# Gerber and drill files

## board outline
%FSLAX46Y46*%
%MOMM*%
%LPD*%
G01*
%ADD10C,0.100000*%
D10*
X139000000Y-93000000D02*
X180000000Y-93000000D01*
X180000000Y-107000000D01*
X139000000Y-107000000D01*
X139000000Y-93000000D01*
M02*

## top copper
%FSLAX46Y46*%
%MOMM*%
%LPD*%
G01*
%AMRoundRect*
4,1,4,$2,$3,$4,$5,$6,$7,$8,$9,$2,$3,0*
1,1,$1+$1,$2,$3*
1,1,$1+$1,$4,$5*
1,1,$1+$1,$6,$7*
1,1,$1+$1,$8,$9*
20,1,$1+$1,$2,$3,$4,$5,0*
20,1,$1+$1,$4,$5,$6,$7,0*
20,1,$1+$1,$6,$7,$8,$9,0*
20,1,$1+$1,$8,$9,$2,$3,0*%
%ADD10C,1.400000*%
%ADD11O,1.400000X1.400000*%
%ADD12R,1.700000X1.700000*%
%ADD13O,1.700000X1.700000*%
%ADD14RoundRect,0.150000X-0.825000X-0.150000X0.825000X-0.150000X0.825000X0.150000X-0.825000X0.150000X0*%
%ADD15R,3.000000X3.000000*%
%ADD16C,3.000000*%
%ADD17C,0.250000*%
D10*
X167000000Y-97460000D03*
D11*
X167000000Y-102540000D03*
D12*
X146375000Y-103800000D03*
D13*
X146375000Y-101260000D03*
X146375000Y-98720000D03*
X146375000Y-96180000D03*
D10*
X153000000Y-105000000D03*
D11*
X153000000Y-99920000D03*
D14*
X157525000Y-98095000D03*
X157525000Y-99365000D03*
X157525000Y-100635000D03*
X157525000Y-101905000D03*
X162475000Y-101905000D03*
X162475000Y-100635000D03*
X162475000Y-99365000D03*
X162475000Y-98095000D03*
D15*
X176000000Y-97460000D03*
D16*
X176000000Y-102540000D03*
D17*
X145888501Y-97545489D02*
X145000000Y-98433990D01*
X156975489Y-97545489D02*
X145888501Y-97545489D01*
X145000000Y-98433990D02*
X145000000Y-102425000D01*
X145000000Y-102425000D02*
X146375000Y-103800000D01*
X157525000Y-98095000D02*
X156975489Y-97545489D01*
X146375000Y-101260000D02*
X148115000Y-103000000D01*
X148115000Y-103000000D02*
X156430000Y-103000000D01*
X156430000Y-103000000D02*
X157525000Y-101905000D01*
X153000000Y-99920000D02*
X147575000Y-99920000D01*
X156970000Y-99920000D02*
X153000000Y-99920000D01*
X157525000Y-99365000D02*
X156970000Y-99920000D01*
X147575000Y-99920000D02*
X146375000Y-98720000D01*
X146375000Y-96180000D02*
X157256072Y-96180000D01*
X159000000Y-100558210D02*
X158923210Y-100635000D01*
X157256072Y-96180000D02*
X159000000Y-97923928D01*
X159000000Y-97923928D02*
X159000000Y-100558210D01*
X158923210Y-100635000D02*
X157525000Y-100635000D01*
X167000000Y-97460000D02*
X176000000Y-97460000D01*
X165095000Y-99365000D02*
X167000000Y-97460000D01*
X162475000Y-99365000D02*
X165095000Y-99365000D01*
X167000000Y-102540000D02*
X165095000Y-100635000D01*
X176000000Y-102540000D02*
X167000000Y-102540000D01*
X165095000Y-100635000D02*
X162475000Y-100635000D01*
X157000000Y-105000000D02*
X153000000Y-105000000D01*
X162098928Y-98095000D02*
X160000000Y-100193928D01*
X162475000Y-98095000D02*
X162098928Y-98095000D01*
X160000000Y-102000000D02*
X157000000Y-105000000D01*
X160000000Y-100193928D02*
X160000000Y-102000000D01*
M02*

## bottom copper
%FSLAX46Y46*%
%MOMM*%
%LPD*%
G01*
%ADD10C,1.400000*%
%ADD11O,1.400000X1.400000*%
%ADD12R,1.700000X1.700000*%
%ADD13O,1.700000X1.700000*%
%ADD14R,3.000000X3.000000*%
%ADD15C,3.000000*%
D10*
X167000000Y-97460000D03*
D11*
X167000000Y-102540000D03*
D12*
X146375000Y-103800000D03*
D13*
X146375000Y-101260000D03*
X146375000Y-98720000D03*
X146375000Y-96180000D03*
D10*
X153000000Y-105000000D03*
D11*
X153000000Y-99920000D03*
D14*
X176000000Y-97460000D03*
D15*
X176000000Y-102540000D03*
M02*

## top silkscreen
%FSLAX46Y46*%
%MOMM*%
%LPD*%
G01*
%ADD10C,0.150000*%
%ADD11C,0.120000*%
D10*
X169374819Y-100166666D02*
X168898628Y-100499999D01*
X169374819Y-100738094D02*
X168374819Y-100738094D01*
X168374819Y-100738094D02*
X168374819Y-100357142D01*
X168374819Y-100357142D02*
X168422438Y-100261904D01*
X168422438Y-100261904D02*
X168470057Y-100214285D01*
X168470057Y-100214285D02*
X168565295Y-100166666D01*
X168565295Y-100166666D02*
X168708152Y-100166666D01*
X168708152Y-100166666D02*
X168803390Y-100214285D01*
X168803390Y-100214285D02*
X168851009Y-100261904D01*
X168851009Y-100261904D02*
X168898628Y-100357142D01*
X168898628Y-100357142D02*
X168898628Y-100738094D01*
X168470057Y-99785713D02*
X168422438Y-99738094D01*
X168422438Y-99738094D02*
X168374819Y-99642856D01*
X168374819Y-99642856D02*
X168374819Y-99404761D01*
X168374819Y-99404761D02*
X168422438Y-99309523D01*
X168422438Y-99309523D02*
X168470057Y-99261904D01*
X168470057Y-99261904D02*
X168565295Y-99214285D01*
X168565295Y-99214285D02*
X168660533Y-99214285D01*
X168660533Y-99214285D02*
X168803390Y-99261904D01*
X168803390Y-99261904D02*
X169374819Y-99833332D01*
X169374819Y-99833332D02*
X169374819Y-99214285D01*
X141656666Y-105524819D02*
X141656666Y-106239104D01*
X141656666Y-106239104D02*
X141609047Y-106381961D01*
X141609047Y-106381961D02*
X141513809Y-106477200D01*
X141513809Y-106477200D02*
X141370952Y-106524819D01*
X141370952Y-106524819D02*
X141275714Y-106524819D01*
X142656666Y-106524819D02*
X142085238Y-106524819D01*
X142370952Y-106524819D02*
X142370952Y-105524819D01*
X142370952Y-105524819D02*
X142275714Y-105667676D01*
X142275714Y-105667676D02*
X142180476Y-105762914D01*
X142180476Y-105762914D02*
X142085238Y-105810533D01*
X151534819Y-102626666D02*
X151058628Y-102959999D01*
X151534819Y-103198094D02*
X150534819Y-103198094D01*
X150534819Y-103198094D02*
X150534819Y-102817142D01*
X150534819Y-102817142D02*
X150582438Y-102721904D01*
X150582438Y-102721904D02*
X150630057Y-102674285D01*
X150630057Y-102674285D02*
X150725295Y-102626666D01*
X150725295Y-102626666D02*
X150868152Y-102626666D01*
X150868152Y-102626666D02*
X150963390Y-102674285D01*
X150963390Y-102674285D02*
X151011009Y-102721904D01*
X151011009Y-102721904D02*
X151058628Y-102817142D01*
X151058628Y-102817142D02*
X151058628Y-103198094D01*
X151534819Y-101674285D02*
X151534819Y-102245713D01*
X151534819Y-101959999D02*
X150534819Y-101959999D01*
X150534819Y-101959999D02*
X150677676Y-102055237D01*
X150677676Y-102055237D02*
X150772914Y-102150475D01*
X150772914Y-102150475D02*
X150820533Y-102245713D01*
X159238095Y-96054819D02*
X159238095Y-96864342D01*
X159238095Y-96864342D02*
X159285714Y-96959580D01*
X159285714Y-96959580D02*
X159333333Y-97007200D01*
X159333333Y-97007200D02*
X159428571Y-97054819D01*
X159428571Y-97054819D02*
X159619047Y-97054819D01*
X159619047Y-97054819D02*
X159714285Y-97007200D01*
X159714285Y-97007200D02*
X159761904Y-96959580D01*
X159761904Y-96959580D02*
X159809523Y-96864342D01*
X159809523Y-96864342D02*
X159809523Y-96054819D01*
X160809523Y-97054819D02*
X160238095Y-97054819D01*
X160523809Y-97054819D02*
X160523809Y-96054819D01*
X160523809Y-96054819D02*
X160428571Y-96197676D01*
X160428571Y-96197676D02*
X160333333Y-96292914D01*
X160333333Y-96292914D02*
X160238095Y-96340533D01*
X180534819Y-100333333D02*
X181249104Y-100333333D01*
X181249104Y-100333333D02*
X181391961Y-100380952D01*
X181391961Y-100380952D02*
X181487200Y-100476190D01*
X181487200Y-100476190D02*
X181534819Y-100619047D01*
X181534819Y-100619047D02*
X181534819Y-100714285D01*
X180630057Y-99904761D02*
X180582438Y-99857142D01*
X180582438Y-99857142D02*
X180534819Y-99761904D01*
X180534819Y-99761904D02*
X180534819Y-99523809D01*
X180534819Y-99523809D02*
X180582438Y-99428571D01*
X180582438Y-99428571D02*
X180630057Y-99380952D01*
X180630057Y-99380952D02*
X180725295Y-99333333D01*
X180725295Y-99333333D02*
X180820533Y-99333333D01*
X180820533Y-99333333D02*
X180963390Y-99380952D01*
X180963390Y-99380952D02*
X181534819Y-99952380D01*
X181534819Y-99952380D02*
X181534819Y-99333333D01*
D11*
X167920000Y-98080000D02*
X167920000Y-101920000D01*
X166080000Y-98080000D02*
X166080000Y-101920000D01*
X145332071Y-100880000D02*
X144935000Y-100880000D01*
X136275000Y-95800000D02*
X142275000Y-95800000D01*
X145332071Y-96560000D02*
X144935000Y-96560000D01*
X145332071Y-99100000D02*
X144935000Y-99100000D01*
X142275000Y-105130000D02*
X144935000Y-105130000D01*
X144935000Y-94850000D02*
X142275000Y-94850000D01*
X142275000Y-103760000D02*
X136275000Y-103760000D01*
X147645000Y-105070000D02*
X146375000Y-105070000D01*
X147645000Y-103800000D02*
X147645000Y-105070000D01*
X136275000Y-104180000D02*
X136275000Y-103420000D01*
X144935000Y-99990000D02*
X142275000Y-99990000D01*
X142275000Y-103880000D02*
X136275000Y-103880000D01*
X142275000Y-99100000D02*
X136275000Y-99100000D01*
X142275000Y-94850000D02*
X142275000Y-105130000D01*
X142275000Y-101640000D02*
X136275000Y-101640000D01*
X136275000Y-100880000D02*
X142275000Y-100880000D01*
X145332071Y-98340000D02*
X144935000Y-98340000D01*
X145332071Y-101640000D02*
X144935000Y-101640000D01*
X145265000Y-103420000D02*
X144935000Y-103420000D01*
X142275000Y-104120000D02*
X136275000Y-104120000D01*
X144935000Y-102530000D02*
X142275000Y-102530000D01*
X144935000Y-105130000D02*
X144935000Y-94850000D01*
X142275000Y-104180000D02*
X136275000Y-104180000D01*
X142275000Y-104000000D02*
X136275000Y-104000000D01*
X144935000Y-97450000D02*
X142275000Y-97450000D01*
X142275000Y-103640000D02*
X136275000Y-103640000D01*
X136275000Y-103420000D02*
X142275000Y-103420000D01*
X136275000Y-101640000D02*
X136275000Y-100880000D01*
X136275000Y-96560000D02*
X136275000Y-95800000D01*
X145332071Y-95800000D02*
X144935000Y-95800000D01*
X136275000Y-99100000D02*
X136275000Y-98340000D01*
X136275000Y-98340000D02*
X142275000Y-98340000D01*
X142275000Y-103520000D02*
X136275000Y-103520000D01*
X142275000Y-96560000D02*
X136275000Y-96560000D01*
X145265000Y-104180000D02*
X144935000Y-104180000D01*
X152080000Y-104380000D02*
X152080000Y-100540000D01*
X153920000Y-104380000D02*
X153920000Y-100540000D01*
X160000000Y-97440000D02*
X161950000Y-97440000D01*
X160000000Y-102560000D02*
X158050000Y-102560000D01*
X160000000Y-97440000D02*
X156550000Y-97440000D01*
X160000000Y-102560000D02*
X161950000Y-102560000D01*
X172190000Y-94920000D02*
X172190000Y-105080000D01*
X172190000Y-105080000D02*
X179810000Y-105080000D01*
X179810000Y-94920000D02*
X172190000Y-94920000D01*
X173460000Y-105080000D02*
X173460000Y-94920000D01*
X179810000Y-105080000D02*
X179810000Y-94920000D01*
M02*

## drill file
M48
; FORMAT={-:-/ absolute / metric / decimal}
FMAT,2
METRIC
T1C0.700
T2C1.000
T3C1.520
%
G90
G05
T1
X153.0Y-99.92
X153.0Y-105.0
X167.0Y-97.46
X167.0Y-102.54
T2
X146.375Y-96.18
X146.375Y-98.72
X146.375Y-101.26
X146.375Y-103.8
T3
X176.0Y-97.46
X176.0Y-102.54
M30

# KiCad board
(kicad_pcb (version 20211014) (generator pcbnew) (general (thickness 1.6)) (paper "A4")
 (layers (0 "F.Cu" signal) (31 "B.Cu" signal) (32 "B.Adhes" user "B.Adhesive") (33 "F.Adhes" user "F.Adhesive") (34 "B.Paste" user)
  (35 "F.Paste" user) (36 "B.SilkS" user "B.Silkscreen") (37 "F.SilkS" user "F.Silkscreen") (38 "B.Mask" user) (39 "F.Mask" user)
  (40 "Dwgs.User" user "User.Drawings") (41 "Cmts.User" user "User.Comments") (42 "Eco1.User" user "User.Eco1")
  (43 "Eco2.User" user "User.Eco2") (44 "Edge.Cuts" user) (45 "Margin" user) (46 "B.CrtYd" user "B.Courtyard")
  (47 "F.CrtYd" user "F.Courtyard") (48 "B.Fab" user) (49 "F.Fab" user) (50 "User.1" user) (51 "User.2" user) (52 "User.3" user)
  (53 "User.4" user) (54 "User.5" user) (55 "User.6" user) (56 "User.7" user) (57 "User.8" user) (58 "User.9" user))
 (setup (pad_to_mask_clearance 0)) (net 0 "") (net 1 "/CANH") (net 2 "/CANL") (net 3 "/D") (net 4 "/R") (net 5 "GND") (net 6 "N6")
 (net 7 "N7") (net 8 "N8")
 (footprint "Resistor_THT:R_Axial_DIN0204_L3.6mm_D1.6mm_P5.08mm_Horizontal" (layer "F.Cu") (at 167 97.46 -90)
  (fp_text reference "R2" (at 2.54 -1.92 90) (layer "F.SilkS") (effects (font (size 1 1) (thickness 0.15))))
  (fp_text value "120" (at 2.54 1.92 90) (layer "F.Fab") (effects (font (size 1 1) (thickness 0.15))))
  (fp_line (start 0.62 -0.92) (end 4.46 -0.92) (layer "F.SilkS") (width 0.12))
  (fp_line (start 0.62 0.92) (end 4.46 0.92) (layer "F.SilkS") (width 0.12))
  (pad "1" thru_hole circle (at 0 0 270) (size 1.4 1.4) (drill 0.7) (layers *.Cu *.Mask) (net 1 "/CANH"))
  (pad "2" thru_hole oval (at 5.08 0 270) (size 1.4 1.4) (drill 0.7) (layers *.Cu *.Mask) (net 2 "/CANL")))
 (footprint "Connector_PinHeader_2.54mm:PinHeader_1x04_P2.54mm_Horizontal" (layer "F.Cu") (at 146.375 103.8 180)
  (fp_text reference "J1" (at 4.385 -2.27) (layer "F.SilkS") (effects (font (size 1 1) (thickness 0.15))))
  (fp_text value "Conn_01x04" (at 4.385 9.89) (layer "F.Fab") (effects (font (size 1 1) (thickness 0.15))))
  (fp_line (start 1.042929 2.92) (end 1.44 2.92) (layer "F.SilkS") (width 0.12))
  (fp_line (start 10.1 8) (end 4.1 8) (layer "F.SilkS") (width 0.12))
  (fp_line (start 1.042929 7.24) (end 1.44 7.24) (layer "F.SilkS") (width 0.12))
  (fp_line (start 1.042929 4.7) (end 1.44 4.7) (layer "F.SilkS") (width 0.12))
  (fp_line (start 4.1 -1.33) (end 1.44 -1.33) (layer "F.SilkS") (width 0.12))
  (fp_line (start 1.44 8.95) (end 4.1 8.95) (layer "F.SilkS") (width 0.12))
  (fp_line (start 4.1 0.04) (end 10.1 0.04) (layer "F.SilkS") (width 0.12))
  (fp_line (start -1.27 -1.27) (end 0 -1.27) (layer "F.SilkS") (width 0.12))
  (fp_line (start -1.27 0) (end -1.27 -1.27) (layer "F.SilkS") (width 0.12))
  (fp_line (start 10.1 -0.38) (end 10.1 0.38) (layer "F.SilkS") (width 0.12))
  (fp_line (start 1.44 3.81) (end 4.1 3.81) (layer "F.SilkS") (width 0.12))
  (fp_line (start 4.1 -0.08) (end 10.1 -0.08) (layer "F.SilkS") (width 0.12))
  (fp_line (start 4.1 4.7) (end 10.1 4.7) (layer "F.SilkS") (width 0.12))
  (fp_line (start 4.1 8.95) (end 4.1 -1.33) (layer "F.SilkS") (width 0.12))
  (fp_line (start 4.1 2.16) (end 10.1 2.16) (layer "F.SilkS") (width 0.12))
  (fp_line (start 10.1 2.92) (end 4.1 2.92) (layer "F.SilkS") (width 0.12))
  (fp_line (start 1.042929 5.46) (end 1.44 5.46) (layer "F.SilkS") (width 0.12))
  (fp_line (start 1.042929 2.16) (end 1.44 2.16) (layer "F.SilkS") (width 0.12))
  (fp_line (start 1.11 0.38) (end 1.44 0.38) (layer "F.SilkS") (width 0.12))
  (fp_line (start 4.1 -0.32) (end 10.1 -0.32) (layer "F.SilkS") (width 0.12))
  (fp_line (start 1.44 1.27) (end 4.1 1.27) (layer "F.SilkS") (width 0.12))
  (fp_line (start 1.44 -1.33) (end 1.44 8.95) (layer "F.SilkS") (width 0.12))
  (fp_line (start 4.1 -0.38) (end 10.1 -0.38) (layer "F.SilkS") (width 0.12))
  (fp_line (start 4.1 -0.2) (end 10.1 -0.2) (layer "F.SilkS") (width 0.12))
  (fp_line (start 1.44 6.35) (end 4.1 6.35) (layer "F.SilkS") (width 0.12))
  (fp_line (start 4.1 0.16) (end 10.1 0.16) (layer "F.SilkS") (width 0.12))
  (fp_line (start 10.1 0.38) (end 4.1 0.38) (layer "F.SilkS") (width 0.12))
  (fp_line (start 10.1 2.16) (end 10.1 2.92) (layer "F.SilkS") (width 0.12))
  (fp_line (start 10.1 7.24) (end 10.1 8) (layer "F.SilkS") (width 0.12))
  (fp_line (start 1.042929 8) (end 1.44 8) (layer "F.SilkS") (width 0.12))
  (fp_line (start 10.1 4.7) (end 10.1 5.46) (layer "F.SilkS") (width 0.12))
  (fp_line (start 10.1 5.46) (end 4.1 5.46) (layer "F.SilkS") (width 0.12))
  (fp_line (start 4.1 0.28) (end 10.1 0.28) (layer "F.SilkS") (width 0.12))
  (fp_line (start 4.1 7.24) (end 10.1 7.24) (layer "F.SilkS") (width 0.12))
  (fp_line (start 1.11 -0.38) (end 1.44 -0.38) (layer "F.SilkS") (width 0.12))
  (pad "1" thru_hole rect (at 0 0 180) (size 1.7 1.7) (drill 1) (layers *.Cu *.Mask) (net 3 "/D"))
  (pad "2" thru_hole oval (at 0 2.54 180) (size 1.7 1.7) (drill 1) (layers *.Cu *.Mask) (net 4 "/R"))
  (pad "3" thru_hole oval (at 0 5.08 180) (size 1.7 1.7) (drill 1) (layers *.Cu *.Mask) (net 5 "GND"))
  (pad "4" thru_hole oval (at 0 7.62 180) (size 1.7 1.7) (drill 1) (layers *.Cu *.Mask) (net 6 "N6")))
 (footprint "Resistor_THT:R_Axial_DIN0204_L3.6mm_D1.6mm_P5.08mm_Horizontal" (layer "F.Cu") (at 153 105 90)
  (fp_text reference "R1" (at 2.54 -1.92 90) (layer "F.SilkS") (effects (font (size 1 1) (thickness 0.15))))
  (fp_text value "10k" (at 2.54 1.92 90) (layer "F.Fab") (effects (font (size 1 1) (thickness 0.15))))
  (fp_line (start 0.62 -0.92) (end 4.46 -0.92) (layer "F.SilkS") (width 0.12))
  (fp_line (start 0.62 0.92) (end 4.46 0.92) (layer "F.SilkS") (width 0.12))
  (pad "1" thru_hole circle (at 0 0 90) (size 1.4 1.4) (drill 0.7) (layers *.Cu *.Mask) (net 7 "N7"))
  (pad "2" thru_hole oval (at 5.08 0 90) (size 1.4 1.4) (drill 0.7) (layers *.Cu *.Mask) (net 5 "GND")))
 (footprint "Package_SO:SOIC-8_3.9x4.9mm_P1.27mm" (layer "F.Cu") (at 160 100)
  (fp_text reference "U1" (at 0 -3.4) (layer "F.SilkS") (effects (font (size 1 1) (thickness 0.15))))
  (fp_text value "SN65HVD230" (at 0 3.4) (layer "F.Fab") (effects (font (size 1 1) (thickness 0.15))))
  (fp_line (start 0 -2.56) (end 1.95 -2.56) (layer "F.SilkS") (width 0.12))
  (fp_line (start 0 2.56) (end -1.95 2.56) (layer "F.SilkS") (width 0.12))
  (fp_line (start 0 -2.56) (end -3.45 -2.56) (layer "F.SilkS") (width 0.12))
  (fp_line (start 0 2.56) (end 1.95 2.56) (layer "F.SilkS") (width 0.12))
  (pad "1" smd roundrect (at -2.475 -1.905) (size 1.95 0.6) (layers "F.Cu" "F.Paste" "F.Mask") (roundrect_rratio 0.25) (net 3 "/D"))
  (pad "2" smd roundrect (at -2.475 -0.635) (size 1.95 0.6) (layers "F.Cu" "F.Paste" "F.Mask") (roundrect_rratio 0.25) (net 5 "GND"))
  (pad "3" smd roundrect (at -2.475 0.635) (size 1.95 0.6) (layers "F.Cu" "F.Paste" "F.Mask") (roundrect_rratio 0.25) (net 6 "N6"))
  (pad "4" smd roundrect (at -2.475 1.905) (size 1.95 0.6) (layers "F.Cu" "F.Paste" "F.Mask") (roundrect_rratio 0.25) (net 4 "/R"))
  (pad "5" smd roundrect (at 2.475 1.905) (size 1.95 0.6) (layers "F.Cu" "F.Paste" "F.Mask") (roundrect_rratio 0.25) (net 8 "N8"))
  (pad "6" smd roundrect (at 2.475 0.635) (size 1.95 0.6) (layers "F.Cu" "F.Paste" "F.Mask") (roundrect_rratio 0.25) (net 2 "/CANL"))
  (pad "7" smd roundrect (at 2.475 -0.635) (size 1.95 0.6) (layers "F.Cu" "F.Paste" "F.Mask") (roundrect_rratio 0.25) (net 1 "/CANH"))
  (pad "8" smd roundrect (at 2.475 -1.905) (size 1.95 0.6) (layers "F.Cu" "F.Paste" "F.Mask") (roundrect_rratio 0.25) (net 7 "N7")))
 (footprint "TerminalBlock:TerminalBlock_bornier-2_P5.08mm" (layer "F.Cu") (at 176 97.46 -90)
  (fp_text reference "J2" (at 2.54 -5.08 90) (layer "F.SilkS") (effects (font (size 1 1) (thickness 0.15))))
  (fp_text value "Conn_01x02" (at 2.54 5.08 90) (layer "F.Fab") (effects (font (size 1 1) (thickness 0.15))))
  (fp_line (start -2.54 3.81) (end 7.62 3.81) (layer "F.SilkS") (width 0.12))
  (fp_line (start 7.62 3.81) (end 7.62 -3.81) (layer "F.SilkS") (width 0.12))
  (fp_line (start -2.54 -3.81) (end -2.54 3.81) (layer "F.SilkS") (width 0.12))
  (fp_line (start 7.62 2.54) (end -2.54 2.54) (layer "F.SilkS") (width 0.12))
  (fp_line (start 7.62 -3.81) (end -2.54 -3.81) (layer "F.SilkS") (width 0.12))
  (pad "1" thru_hole rect (at 0 0 270) (size 3 3) (drill 1.52) (layers *.Cu *.Mask) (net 1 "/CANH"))
  (pad "2" thru_hole circle (at 5.08 0 270) (size 3 3) (drill 1.52) (layers *.Cu *.Mask) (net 2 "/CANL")))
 (gr_rect (start 180 107) (end 139 93) (layer "Edge.Cuts") (width 0.1) (fill none))
 (segment (start 145.888501 97.545489) (end 145 98.43399) (width 0.25) (layer "F.Cu") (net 3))
 (segment (start 156.975489 97.545489) (end 145.888501 97.545489) (width 0.25) (layer "F.Cu") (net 3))
 (segment (start 145 98.43399) (end 145 102.425) (width 0.25) (layer "F.Cu") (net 3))
 (segment (start 145 102.425) (end 146.375 103.8) (width 0.25) (layer "F.Cu") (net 3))
 (segment (start 157.525 98.095) (end 156.975489 97.545489) (width 0.25) (layer "F.Cu") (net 3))
 (segment (start 146.375 101.26) (end 148.115 103) (width 0.25) (layer "F.Cu") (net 4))
 (segment (start 148.115 103) (end 156.43 103) (width 0.25) (layer "F.Cu") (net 4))
 (segment (start 156.43 103) (end 157.525 101.905) (width 0.25) (layer "F.Cu") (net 4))
 (segment (start 153 99.92) (end 147.575 99.92) (width 0.25) (layer "F.Cu") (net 5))
 (segment (start 156.97 99.92) (end 153 99.92) (width 0.25) (layer "F.Cu") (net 5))
 (segment (start 157.525 99.365) (end 156.97 99.92) (width 0.25) (layer "F.Cu") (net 5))
 (segment (start 147.575 99.92) (end 146.375 98.72) (width 0.25) (layer "F.Cu") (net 5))
 (segment (start 146.375 96.18) (end 157.256072 96.18) (width 0.25) (layer "F.Cu") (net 6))
 (segment (start 159 100.55821) (end 158.92321 100.635) (width 0.25) (layer "F.Cu") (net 6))
 (segment (start 157.256072 96.18) (end 159 97.923928) (width 0.25) (layer "F.Cu") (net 6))
 (segment (start 159 97.923928) (end 159 100.55821) (width 0.25) (layer "F.Cu") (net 6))
 (segment (start 158.92321 100.635) (end 157.525 100.635) (width 0.25) (layer "F.Cu") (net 6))
 (segment (start 167 97.46) (end 176 97.46) (width 0.25) (layer "F.Cu") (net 1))
 (segment (start 165.095 99.365) (end 167 97.46) (width 0.25) (layer "F.Cu") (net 1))
 (segment (start 162.475 99.365) (end 165.095 99.365) (width 0.25) (layer "F.Cu") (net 1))
 (segment (start 167 102.54) (end 165.095 100.635) (width 0.25) (layer "F.Cu") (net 2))
 (segment (start 176 102.54) (end 167 102.54) (width 0.25) (layer "F.Cu") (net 2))
 (segment (start 165.095 100.635) (end 162.475 100.635) (width 0.25) (layer "F.Cu") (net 2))
 (segment (start 157 105) (end 153 105) (width 0.25) (layer "F.Cu") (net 7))
 (segment (start 162.098928 98.095) (end 160 100.193928) (width 0.25) (layer "F.Cu") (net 7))
 (segment (start 162.475 98.095) (end 162.098928 98.095) (width 0.25) (layer "F.Cu") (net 7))
 (segment (start 160 102) (end 157 105) (width 0.25) (layer "F.Cu") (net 7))
 (segment (start 160 100.193928) (end 160 102) (width 0.25) (layer "F.Cu") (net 7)))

